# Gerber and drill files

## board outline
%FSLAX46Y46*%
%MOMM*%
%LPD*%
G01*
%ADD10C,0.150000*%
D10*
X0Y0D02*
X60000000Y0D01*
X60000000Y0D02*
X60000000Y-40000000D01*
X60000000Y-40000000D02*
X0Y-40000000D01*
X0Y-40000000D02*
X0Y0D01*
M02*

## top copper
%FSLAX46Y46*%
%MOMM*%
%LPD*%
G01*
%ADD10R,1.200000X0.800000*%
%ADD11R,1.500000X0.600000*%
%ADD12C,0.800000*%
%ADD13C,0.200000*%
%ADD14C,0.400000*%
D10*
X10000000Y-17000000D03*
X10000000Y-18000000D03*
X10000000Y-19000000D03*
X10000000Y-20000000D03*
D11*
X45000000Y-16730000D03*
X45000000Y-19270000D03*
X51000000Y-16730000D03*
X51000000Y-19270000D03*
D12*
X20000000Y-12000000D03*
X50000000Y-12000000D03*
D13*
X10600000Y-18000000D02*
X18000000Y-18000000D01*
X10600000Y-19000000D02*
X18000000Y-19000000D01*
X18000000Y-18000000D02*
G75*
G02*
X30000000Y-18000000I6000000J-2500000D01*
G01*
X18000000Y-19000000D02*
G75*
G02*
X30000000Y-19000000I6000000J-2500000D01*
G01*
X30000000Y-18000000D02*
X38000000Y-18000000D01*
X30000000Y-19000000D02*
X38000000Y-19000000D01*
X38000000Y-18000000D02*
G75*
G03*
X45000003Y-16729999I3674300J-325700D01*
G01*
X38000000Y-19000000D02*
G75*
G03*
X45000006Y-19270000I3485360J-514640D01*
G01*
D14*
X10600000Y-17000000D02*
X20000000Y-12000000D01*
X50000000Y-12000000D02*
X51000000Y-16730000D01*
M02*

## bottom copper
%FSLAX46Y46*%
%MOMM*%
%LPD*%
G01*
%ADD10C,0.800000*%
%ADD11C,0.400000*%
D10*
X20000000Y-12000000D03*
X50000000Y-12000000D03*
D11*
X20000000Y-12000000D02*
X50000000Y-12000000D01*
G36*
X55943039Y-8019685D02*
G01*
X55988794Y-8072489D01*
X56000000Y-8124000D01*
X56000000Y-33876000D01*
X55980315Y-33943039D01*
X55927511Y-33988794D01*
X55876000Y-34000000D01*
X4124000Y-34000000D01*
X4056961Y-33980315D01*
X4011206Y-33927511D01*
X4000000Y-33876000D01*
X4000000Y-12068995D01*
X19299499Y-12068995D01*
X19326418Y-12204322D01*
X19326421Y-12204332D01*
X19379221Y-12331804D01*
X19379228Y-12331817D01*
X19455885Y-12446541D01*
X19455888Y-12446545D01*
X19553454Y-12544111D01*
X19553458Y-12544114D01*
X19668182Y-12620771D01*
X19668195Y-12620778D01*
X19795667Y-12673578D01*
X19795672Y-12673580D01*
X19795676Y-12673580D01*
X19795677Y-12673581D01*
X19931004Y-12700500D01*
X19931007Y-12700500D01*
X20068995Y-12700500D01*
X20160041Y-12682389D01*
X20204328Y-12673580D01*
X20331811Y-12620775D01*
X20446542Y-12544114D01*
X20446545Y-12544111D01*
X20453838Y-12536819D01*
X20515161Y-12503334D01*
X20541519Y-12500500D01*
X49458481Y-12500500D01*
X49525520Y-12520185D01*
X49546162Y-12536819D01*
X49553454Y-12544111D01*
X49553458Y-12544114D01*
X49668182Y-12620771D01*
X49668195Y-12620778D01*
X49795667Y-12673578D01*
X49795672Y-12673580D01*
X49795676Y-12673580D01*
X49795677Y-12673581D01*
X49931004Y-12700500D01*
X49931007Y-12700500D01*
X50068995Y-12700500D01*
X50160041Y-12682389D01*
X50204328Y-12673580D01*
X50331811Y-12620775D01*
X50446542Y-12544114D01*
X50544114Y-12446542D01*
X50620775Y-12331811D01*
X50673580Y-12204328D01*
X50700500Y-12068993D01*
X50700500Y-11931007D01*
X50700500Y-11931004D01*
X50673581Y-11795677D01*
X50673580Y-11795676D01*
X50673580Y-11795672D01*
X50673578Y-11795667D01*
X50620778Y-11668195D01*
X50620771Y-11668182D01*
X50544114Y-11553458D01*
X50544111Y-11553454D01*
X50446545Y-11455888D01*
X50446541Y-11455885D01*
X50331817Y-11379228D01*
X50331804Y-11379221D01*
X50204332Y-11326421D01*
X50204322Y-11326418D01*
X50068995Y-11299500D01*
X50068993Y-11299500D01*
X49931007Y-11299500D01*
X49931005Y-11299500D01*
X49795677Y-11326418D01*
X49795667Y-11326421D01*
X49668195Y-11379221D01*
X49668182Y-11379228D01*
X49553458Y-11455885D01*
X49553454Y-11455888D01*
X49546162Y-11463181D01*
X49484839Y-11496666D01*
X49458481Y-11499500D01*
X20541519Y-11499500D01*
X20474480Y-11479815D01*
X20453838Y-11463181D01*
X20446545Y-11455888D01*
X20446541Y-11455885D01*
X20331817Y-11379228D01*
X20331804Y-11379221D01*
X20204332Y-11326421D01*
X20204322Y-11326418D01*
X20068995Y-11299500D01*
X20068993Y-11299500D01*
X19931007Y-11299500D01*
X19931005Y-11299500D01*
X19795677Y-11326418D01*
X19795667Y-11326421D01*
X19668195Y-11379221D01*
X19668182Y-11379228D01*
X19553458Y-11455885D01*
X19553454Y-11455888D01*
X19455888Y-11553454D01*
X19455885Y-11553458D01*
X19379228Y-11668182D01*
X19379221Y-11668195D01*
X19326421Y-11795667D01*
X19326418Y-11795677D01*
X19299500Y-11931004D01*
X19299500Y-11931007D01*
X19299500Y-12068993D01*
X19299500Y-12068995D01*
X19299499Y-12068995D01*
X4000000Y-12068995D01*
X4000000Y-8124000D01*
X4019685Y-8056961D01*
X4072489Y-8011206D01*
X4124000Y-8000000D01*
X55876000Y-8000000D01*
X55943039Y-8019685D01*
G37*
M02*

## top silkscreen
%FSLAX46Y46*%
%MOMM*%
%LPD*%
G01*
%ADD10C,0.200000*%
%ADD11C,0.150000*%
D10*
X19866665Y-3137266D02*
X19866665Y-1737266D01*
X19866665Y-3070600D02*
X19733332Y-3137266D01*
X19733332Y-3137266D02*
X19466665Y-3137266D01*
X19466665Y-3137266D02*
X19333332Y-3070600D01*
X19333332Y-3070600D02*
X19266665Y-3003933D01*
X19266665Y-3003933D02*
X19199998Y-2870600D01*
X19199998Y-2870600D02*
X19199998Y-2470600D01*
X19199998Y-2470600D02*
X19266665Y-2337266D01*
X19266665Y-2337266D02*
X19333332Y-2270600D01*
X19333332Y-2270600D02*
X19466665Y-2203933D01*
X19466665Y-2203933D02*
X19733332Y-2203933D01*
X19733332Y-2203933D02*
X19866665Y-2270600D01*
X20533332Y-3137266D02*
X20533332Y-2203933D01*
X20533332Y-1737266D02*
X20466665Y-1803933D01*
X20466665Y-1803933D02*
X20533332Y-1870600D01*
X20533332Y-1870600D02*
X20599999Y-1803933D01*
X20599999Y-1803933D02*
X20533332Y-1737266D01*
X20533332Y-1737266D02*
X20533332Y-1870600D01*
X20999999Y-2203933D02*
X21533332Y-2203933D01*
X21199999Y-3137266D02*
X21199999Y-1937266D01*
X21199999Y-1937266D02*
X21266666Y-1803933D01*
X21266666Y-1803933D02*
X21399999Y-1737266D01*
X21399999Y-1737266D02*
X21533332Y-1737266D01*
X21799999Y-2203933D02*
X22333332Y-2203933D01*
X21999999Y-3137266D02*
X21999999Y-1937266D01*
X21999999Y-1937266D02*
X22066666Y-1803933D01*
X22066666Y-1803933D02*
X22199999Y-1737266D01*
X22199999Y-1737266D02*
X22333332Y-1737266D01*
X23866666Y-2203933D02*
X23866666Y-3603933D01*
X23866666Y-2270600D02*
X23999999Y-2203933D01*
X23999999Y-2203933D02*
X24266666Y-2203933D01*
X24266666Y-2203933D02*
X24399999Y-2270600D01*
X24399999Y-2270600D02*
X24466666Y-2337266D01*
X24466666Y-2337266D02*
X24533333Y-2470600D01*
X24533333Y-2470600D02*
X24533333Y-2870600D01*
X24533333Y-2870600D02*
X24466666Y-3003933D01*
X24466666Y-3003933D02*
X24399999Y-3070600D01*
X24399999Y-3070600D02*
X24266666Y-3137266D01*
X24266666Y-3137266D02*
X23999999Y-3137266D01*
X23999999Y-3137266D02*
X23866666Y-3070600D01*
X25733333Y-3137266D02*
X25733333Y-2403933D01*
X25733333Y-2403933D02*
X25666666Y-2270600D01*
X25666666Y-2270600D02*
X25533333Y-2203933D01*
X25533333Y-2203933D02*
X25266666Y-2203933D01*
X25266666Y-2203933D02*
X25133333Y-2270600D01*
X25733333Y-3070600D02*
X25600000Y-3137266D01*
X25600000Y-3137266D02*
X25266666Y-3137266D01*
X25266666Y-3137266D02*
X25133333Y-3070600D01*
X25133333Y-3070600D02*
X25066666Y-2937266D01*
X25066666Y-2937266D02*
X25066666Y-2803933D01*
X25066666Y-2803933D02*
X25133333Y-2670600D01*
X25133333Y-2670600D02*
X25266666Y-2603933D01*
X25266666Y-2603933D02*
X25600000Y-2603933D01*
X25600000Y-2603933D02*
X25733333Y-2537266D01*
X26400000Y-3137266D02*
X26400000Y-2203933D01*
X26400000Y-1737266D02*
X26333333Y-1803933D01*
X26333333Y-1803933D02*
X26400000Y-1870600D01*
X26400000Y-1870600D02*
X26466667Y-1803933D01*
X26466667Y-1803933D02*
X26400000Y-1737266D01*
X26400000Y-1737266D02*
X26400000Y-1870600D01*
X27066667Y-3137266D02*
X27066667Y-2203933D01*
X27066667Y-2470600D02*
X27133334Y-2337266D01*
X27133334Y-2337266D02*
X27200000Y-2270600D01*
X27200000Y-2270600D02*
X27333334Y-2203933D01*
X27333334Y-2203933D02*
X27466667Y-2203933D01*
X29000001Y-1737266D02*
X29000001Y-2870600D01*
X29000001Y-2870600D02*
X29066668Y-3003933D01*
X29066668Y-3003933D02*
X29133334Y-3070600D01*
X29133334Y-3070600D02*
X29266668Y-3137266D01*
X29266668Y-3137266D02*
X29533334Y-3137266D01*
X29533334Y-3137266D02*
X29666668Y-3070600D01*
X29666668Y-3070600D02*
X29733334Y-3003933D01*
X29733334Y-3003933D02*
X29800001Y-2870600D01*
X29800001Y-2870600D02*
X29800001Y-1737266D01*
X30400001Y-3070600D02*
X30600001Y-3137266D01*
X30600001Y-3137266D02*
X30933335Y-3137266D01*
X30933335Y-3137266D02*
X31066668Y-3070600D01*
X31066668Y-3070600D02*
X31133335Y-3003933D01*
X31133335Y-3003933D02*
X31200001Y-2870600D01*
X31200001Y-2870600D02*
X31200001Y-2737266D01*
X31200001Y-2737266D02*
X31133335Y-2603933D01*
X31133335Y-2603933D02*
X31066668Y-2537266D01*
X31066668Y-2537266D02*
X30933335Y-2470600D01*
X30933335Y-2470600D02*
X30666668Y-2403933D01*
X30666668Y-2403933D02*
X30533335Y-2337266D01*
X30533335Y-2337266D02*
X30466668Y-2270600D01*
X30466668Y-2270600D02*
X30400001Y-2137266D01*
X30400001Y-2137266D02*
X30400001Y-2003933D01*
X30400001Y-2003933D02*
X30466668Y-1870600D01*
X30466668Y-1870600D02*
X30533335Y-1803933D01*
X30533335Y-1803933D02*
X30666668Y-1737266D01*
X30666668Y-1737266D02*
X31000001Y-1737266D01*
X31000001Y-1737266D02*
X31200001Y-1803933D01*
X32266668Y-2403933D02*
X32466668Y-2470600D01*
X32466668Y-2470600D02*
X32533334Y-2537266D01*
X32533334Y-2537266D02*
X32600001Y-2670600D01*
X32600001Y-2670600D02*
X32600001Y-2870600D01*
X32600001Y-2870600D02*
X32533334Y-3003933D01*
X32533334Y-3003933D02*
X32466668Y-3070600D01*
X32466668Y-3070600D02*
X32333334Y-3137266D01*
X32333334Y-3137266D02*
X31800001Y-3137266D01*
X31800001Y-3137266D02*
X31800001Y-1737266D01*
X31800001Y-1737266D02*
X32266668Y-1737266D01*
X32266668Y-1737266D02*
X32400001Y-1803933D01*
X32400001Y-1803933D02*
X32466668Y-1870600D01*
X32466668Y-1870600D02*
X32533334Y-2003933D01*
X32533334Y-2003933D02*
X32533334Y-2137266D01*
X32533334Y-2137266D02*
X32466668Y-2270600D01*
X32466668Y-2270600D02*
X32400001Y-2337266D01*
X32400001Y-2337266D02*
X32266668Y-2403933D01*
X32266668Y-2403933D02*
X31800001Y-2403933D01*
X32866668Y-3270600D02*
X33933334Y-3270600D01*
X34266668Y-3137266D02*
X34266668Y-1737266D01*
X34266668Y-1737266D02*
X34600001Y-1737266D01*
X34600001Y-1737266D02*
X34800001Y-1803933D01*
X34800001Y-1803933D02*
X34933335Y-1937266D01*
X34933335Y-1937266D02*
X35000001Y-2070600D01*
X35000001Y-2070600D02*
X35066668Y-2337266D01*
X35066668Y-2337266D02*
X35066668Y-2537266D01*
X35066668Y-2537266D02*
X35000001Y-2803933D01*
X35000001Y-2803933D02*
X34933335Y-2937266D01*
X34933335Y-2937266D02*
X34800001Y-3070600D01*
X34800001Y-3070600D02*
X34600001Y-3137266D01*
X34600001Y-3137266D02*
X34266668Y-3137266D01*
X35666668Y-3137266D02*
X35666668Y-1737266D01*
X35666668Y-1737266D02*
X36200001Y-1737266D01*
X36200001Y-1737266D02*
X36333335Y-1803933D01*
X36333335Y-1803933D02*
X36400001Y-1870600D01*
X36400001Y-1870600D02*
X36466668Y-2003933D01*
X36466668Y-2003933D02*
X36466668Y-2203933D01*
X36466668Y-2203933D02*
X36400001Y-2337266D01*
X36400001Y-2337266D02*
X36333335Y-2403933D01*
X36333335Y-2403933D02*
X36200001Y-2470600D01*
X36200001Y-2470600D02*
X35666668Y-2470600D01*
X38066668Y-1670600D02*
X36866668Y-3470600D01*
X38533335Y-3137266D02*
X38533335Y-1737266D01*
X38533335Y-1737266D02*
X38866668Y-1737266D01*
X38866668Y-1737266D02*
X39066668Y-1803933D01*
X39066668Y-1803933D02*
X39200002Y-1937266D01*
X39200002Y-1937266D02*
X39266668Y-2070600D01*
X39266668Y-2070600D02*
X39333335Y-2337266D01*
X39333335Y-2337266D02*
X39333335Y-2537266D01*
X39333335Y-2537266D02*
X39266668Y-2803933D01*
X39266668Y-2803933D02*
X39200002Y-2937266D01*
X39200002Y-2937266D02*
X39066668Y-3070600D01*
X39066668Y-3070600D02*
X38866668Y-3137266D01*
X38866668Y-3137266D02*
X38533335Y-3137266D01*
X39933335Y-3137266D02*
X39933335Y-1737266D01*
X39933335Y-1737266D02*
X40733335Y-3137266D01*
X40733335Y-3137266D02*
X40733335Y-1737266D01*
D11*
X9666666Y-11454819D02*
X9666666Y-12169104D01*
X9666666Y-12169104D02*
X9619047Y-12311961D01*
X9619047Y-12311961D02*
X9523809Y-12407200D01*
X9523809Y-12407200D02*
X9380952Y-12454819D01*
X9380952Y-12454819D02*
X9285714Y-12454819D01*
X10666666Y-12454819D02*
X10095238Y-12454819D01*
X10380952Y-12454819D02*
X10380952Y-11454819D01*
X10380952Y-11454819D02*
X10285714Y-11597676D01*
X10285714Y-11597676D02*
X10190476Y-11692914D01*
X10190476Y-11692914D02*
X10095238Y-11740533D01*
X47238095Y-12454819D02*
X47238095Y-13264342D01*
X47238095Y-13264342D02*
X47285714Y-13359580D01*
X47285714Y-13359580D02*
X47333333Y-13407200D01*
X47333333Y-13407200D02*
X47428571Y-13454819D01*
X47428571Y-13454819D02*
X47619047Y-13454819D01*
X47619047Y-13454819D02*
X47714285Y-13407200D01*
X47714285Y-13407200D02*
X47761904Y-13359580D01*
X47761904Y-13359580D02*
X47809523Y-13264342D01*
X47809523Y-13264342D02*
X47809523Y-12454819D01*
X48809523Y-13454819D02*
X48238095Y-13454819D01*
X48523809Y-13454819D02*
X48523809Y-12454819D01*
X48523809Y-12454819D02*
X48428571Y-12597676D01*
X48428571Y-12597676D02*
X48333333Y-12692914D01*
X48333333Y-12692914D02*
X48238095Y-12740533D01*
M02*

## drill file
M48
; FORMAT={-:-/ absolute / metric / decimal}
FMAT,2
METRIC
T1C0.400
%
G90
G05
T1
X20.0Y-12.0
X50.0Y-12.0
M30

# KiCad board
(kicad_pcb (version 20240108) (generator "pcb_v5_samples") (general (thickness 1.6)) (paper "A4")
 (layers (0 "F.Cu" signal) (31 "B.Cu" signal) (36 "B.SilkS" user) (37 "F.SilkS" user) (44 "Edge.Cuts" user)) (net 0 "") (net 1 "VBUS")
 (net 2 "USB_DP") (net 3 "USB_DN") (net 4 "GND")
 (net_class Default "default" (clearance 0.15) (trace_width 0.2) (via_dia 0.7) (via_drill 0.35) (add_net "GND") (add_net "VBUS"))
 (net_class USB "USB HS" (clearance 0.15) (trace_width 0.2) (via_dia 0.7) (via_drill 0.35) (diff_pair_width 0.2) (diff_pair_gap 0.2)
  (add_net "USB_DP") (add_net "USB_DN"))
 (gr_line (start 0 0) (end 60 0) (stroke (width 0.15) (type solid)) (layer "Edge.Cuts"))
 (gr_line (start 60 0) (end 60 40) (stroke (width 0.15) (type solid)) (layer "Edge.Cuts"))
 (gr_line (start 60 40) (end 0 40) (stroke (width 0.15) (type solid)) (layer "Edge.Cuts"))
 (gr_line (start 0 40) (end 0 0) (stroke (width 0.15) (type solid)) (layer "Edge.Cuts"))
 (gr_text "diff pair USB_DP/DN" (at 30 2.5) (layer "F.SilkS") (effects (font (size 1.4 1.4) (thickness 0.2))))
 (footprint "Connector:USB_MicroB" (layer "F.Cu") (at 10 18)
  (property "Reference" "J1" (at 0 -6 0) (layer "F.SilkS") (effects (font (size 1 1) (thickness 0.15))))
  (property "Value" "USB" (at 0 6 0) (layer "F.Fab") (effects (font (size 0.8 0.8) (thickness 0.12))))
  (pad "1" smd rect (at 0 -1.0) (size 1.2 0.8) (layers "F.Cu" "F.Paste" "F.Mask") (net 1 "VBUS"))
  (pad "2" smd rect (at 0 0.0) (size 1.2 0.8) (layers "F.Cu" "F.Paste" "F.Mask") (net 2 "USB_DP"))
  (pad "3" smd rect (at 0 1.0) (size 1.2 0.8) (layers "F.Cu" "F.Paste" "F.Mask") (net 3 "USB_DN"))
  (pad "4" smd rect (at 0 2.0) (size 1.2 0.8) (layers "F.Cu" "F.Paste" "F.Mask") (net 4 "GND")))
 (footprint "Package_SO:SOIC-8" (layer "F.Cu") (at 48 18)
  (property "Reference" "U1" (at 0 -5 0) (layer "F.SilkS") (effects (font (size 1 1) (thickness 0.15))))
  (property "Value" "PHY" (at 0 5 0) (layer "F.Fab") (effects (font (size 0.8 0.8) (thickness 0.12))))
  (pad "1" smd rect (at -3.0 -1.27) (size 1.5 0.6) (layers "F.Cu" "F.Paste" "F.Mask") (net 2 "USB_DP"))
  (pad "2" smd rect (at -3.0 1.27) (size 1.5 0.6) (layers "F.Cu" "F.Paste" "F.Mask") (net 3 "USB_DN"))
  (pad "3" smd rect (at 3.0 -1.27) (size 1.5 0.6) (layers "F.Cu" "F.Paste" "F.Mask") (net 1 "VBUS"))
  (pad "4" smd rect (at 3.0 1.27) (size 1.5 0.6) (layers "F.Cu" "F.Paste" "F.Mask") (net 4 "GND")))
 (segment (start 10.6 18) (end 18 18) (width 0.2) (layer "F.Cu") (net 2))
 (segment (start 10.6 19) (end 18 19) (width 0.2) (layer "F.Cu") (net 3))
 (arc (start 18 18) (mid 24 14) (end 30 18) (width 0.2) (layer "F.Cu") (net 2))
 (arc (start 18 19) (mid 24 15) (end 30 19) (width 0.2) (layer "F.Cu") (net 3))
 (segment (start 30 18) (end 38 18) (width 0.2) (layer "F.Cu") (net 2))
 (segment (start 30 19) (end 38 19) (width 0.2) (layer "F.Cu") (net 3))
 (arc (start 38 18) (mid 42 22) (end 45 16.73) (width 0.2) (layer "F.Cu") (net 2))
 (arc (start 38 19) (mid 42 23) (end 45 19.27) (width 0.2) (layer "F.Cu") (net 3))
 (segment (start 10.6 17) (end 20 12) (width 0.4) (layer "F.Cu") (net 1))
 (via (at 20 12) (size 0.8) (drill 0.4) (layers "F.Cu" "B.Cu") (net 1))
 (segment (start 20 12) (end 50 12) (width 0.4) (layer "B.Cu") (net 1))
 (via (at 50 12) (size 0.8) (drill 0.4) (layers "F.Cu" "B.Cu") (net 1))
 (segment (start 50 12) (end 51 16.73) (width 0.4) (layer "F.Cu") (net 1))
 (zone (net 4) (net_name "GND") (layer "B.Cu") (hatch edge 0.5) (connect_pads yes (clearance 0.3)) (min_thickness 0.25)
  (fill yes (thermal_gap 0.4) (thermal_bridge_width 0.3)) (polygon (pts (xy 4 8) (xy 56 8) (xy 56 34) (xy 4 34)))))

